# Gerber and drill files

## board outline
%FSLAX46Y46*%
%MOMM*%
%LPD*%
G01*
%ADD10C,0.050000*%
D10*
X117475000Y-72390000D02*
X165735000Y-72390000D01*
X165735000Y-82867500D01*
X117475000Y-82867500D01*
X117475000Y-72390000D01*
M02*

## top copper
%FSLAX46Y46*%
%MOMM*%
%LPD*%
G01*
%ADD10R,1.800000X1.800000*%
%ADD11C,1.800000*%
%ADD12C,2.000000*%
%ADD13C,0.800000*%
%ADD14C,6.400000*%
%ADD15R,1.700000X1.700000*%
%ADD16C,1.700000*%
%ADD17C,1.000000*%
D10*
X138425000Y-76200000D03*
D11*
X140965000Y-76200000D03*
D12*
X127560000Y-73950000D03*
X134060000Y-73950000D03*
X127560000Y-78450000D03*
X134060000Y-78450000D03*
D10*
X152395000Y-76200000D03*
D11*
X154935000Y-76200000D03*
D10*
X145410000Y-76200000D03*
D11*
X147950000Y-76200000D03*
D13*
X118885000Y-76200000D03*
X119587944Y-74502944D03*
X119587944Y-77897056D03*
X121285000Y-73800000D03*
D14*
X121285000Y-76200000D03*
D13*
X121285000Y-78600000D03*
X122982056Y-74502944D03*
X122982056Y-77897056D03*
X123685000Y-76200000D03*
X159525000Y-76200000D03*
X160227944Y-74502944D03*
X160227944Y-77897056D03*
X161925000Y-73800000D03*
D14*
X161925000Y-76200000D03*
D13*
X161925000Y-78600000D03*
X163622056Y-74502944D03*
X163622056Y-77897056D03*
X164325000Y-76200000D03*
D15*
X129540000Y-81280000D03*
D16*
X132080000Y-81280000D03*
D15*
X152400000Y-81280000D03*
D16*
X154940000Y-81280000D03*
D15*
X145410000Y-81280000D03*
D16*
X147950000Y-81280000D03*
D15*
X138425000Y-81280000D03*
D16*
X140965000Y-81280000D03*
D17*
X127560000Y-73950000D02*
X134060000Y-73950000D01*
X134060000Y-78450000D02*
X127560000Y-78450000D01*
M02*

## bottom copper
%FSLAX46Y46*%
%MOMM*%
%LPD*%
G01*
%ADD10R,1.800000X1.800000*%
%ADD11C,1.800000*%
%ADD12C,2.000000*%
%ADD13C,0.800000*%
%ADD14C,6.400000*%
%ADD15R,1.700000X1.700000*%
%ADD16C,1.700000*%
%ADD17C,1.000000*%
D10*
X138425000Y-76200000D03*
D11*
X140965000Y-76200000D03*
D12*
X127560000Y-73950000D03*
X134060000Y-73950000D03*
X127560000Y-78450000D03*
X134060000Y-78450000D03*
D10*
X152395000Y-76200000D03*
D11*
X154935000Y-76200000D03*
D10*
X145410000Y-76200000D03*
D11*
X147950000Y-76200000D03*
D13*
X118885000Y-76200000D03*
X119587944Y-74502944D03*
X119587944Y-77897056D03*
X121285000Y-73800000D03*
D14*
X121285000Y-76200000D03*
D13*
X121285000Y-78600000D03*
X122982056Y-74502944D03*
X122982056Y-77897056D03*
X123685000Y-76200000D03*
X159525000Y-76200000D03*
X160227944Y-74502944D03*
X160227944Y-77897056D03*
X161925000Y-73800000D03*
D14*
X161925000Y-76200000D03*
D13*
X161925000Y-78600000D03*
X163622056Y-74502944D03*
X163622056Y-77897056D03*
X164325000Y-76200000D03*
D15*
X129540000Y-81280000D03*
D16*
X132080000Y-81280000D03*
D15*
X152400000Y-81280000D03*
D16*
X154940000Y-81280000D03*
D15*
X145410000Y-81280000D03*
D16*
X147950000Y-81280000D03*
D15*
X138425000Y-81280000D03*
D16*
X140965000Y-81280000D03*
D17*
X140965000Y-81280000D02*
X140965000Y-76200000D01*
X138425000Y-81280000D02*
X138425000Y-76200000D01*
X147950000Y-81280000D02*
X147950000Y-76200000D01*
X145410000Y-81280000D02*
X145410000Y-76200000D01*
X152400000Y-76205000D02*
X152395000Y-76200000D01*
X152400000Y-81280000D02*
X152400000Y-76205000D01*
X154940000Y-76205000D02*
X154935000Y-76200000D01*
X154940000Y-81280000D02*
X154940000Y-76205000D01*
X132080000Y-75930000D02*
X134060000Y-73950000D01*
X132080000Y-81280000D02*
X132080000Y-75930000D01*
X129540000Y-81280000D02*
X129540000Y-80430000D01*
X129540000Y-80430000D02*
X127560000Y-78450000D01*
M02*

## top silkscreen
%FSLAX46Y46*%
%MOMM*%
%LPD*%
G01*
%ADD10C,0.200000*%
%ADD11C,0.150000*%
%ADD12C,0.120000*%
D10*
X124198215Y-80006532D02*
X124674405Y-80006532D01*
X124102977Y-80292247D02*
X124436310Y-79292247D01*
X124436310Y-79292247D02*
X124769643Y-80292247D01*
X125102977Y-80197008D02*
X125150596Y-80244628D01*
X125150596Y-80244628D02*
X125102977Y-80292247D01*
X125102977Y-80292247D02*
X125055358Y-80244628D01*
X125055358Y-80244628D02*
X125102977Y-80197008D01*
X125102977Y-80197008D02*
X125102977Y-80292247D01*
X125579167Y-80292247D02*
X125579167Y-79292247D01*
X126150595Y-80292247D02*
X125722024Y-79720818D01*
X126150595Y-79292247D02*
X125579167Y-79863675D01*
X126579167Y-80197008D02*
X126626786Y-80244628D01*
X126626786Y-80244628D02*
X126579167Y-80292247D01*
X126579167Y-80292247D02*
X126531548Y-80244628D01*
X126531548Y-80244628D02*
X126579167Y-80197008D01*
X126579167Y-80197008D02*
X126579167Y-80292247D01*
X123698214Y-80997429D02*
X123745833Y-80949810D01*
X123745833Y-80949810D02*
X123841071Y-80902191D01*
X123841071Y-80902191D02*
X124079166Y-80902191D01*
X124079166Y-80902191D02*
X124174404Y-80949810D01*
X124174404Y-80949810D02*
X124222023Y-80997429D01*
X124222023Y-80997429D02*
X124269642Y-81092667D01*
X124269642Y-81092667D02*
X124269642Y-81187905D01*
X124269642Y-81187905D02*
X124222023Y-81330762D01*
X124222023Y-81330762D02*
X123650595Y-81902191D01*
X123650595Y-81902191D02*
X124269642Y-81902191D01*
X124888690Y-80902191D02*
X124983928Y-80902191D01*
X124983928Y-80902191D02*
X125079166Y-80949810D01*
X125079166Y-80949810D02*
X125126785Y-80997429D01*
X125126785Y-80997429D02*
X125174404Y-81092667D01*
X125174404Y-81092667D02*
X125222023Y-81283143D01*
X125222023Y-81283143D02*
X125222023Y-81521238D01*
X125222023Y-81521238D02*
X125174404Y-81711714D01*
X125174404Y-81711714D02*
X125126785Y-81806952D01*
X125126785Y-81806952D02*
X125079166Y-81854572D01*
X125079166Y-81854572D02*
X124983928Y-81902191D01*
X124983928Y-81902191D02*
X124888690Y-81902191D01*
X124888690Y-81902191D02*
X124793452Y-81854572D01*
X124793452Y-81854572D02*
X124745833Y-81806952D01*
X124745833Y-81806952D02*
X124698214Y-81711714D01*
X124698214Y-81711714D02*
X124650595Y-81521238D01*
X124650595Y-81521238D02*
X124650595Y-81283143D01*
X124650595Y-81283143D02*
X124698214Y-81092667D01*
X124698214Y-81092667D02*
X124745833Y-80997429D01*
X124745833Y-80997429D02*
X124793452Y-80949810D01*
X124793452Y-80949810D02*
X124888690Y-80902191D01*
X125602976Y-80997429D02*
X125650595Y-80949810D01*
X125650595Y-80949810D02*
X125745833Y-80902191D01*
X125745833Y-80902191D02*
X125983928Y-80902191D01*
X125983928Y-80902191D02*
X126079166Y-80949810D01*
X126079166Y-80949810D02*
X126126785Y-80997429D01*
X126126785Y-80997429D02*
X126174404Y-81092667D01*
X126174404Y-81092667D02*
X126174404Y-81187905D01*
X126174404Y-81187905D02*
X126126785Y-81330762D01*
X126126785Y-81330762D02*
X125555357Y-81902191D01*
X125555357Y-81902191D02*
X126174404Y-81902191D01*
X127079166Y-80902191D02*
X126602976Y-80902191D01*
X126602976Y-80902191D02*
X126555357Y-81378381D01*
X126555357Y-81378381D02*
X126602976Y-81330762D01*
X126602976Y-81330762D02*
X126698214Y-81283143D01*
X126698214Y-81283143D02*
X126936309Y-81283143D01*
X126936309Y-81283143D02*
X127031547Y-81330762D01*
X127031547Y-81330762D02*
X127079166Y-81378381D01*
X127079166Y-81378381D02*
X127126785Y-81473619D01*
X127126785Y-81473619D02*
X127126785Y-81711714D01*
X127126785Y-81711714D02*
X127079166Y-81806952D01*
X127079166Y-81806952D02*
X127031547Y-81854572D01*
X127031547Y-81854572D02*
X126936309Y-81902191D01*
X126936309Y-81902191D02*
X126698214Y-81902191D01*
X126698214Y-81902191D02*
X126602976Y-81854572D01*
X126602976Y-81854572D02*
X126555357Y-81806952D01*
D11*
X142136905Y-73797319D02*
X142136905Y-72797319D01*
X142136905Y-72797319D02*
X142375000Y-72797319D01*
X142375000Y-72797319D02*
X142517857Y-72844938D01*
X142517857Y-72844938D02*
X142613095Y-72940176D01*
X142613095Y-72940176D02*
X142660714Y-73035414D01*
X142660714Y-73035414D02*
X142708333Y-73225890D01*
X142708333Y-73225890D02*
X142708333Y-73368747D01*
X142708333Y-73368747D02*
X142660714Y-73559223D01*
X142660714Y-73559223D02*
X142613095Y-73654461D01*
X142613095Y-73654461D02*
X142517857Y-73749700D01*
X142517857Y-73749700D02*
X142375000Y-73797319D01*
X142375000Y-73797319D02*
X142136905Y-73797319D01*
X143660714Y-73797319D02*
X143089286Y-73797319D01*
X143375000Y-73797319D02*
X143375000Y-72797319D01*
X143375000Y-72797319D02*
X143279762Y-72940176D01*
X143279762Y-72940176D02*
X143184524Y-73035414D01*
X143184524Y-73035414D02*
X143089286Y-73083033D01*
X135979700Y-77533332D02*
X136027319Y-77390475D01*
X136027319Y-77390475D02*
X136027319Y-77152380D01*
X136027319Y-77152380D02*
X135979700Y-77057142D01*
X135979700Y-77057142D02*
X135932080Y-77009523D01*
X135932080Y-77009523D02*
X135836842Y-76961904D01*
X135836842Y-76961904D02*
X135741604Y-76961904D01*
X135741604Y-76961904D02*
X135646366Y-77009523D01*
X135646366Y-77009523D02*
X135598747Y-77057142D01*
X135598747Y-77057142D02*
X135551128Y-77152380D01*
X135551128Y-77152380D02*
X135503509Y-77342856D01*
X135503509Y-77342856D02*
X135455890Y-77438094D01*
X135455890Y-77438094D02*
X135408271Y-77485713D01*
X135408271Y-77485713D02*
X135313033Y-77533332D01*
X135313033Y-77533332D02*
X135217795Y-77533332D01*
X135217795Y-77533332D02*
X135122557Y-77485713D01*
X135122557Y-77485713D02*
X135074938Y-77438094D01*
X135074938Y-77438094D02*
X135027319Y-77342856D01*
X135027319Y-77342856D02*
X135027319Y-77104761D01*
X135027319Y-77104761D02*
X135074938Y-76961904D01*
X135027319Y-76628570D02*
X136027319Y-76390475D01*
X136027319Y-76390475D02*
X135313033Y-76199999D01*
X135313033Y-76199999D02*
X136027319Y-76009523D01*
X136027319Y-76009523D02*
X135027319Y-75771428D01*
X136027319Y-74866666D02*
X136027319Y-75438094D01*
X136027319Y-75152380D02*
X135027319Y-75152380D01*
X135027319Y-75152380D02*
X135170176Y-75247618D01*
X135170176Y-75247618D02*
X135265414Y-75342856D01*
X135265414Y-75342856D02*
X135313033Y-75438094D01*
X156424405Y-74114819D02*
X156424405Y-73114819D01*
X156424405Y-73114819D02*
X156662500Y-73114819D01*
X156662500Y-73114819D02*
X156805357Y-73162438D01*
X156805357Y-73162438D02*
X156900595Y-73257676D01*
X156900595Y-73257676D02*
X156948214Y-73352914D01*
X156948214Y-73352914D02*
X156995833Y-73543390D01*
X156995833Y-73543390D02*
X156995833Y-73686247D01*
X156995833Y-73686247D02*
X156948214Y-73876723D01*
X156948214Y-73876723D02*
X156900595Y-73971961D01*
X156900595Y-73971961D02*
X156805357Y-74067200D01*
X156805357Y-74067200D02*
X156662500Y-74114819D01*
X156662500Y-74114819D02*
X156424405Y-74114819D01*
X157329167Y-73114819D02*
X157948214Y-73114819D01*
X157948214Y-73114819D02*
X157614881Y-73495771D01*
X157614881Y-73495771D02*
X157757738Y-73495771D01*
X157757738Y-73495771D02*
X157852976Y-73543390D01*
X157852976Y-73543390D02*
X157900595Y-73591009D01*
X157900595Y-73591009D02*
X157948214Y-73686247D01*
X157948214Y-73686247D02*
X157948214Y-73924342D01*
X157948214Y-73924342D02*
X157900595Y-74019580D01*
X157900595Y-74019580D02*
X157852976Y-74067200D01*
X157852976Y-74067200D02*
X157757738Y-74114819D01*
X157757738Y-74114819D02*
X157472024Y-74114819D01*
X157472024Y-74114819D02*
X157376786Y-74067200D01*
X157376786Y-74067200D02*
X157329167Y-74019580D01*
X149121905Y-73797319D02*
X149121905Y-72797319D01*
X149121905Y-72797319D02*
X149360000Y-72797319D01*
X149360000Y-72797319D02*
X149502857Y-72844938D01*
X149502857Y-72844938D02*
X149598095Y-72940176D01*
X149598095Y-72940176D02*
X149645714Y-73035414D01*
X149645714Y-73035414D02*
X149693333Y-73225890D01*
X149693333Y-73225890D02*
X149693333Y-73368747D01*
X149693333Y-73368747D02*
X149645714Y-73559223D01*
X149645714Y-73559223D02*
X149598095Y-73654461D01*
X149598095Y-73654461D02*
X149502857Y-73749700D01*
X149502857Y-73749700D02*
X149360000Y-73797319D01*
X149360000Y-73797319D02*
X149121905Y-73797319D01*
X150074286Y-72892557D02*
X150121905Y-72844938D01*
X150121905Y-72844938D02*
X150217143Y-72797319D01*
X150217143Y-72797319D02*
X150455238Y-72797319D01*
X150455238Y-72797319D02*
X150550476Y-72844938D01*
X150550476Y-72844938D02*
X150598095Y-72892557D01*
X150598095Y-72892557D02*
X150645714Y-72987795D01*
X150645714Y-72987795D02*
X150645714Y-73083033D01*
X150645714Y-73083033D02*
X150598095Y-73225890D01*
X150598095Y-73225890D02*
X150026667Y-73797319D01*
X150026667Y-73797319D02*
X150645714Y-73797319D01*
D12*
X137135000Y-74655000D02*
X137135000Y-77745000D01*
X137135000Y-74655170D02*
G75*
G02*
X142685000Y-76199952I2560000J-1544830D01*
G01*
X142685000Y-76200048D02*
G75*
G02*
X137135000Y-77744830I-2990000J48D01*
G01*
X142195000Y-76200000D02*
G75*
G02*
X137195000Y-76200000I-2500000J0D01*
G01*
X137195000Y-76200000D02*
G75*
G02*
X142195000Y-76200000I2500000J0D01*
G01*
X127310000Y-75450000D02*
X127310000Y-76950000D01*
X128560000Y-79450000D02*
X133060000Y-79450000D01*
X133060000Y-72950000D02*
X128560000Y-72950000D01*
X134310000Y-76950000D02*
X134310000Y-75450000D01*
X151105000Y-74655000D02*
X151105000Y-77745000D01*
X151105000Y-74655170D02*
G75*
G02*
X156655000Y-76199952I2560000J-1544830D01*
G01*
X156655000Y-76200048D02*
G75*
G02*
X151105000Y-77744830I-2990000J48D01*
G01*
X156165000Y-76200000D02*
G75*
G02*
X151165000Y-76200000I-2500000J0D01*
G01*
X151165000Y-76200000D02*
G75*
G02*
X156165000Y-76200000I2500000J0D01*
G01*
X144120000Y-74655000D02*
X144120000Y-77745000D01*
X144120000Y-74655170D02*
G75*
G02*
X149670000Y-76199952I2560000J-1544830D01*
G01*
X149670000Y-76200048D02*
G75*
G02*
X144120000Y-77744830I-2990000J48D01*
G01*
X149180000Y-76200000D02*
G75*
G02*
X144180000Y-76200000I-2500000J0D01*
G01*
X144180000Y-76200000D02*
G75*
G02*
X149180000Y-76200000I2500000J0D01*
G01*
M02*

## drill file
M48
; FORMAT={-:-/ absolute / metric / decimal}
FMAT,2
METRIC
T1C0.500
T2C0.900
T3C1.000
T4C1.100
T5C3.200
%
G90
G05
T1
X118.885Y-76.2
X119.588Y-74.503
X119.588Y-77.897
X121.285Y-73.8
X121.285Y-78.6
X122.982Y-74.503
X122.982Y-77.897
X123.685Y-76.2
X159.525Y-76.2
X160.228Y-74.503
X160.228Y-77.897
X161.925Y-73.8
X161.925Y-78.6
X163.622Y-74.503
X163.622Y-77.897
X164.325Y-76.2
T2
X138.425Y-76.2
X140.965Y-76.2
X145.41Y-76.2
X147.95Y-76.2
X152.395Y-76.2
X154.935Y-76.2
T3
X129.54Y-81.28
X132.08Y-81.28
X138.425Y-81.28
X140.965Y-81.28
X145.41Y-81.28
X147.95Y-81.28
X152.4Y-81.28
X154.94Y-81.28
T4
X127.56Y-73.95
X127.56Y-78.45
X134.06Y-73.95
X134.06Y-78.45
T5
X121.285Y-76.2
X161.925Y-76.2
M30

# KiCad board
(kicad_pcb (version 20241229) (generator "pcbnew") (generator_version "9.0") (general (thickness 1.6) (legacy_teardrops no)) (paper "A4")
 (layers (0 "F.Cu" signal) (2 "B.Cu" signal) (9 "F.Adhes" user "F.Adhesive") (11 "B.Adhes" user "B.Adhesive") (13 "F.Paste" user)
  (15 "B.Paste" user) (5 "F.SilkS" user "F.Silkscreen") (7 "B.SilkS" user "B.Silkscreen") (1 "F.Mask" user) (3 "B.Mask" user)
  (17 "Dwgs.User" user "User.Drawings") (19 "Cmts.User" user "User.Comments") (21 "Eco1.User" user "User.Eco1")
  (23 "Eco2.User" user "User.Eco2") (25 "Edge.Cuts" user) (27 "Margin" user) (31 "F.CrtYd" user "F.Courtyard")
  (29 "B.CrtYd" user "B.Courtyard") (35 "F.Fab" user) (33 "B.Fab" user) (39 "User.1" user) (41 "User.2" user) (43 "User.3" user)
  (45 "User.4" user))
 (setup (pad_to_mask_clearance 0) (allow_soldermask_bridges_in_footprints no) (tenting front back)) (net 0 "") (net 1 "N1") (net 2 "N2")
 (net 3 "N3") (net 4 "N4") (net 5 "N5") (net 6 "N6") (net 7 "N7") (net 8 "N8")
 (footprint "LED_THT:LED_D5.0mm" (layer "F.Cu") (at 138.425 76.2)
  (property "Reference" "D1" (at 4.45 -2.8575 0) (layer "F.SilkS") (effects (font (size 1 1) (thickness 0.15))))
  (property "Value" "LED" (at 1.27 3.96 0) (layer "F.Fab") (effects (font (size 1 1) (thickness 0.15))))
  (fp_line (start -1.29 -1.545) (end -1.29 1.545) (stroke (width 0.12) (type solid)) (layer "F.SilkS"))
  (fp_arc (start -1.29 -1.54483) (mid 2.071756 -2.880501) (end 4.26 -0.000048) (stroke (width 0.12) (type solid)) (layer "F.SilkS"))
  (fp_arc (start 4.26 0.000048) (mid 2.071756 2.880501) (end -1.29 1.54483) (stroke (width 0.12) (type solid)) (layer "F.SilkS"))
  (fp_circle (center 1.27 0) (end 3.77 0) (stroke (width 0.12) (type solid)) (fill no) (layer "F.SilkS"))
  (pad "1" thru_hole rect (at 0 0) (size 1.8 1.8) (drill 0.9) (layers "*.Cu" "*.Mask") (remove_unused_layers no) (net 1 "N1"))
  (pad "2" thru_hole circle (at 2.54 0) (size 1.8 1.8) (drill 0.9) (layers "*.Cu" "*.Mask") (remove_unused_layers no) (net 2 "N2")))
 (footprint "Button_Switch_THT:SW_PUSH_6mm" (layer "F.Cu") (at 127.56 73.95)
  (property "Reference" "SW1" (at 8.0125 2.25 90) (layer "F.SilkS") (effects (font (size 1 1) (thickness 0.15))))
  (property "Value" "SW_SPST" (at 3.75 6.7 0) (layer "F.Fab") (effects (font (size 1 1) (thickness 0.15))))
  (fp_line (start -0.25 1.5) (end -0.25 3) (stroke (width 0.12) (type solid)) (layer "F.SilkS"))
  (fp_line (start 1 5.5) (end 5.5 5.5) (stroke (width 0.12) (type solid)) (layer "F.SilkS"))
  (fp_line (start 5.5 -1) (end 1 -1) (stroke (width 0.12) (type solid)) (layer "F.SilkS"))
  (fp_line (start 6.75 3) (end 6.75 1.5) (stroke (width 0.12) (type solid)) (layer "F.SilkS"))
  (pad "1" thru_hole circle (at 0 0 90) (size 2 2) (drill 1.1) (layers "*.Cu" "*.Mask") (remove_unused_layers no) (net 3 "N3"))
  (pad "1" thru_hole circle (at 6.5 0 90) (size 2 2) (drill 1.1) (layers "*.Cu" "*.Mask") (remove_unused_layers no) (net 3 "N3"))
  (pad "2" thru_hole circle (at 0 4.5 90) (size 2 2) (drill 1.1) (layers "*.Cu" "*.Mask") (remove_unused_layers no) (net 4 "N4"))
  (pad "2" thru_hole circle (at 6.5 4.5 90) (size 2 2) (drill 1.1) (layers "*.Cu" "*.Mask") (remove_unused_layers no) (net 4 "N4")))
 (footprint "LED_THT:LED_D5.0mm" (layer "F.Cu") (at 152.395 76.2)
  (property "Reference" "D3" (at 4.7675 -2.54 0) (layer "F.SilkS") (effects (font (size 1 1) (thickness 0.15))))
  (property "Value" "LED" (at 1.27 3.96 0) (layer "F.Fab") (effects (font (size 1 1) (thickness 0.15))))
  (fp_line (start -1.29 -1.545) (end -1.29 1.545) (stroke (width 0.12) (type solid)) (layer "F.SilkS"))
  (fp_arc (start -1.29 -1.54483) (mid 2.071756 -2.880501) (end 4.26 -0.000048) (stroke (width 0.12) (type solid)) (layer "F.SilkS"))
  (fp_arc (start 4.26 0.000048) (mid 2.071756 2.880501) (end -1.29 1.54483) (stroke (width 0.12) (type solid)) (layer "F.SilkS"))
  (fp_circle (center 1.27 0) (end 3.77 0) (stroke (width 0.12) (type solid)) (fill no) (layer "F.SilkS"))
  (pad "1" thru_hole rect (at 0 0) (size 1.8 1.8) (drill 0.9) (layers "*.Cu" "*.Mask") (remove_unused_layers no) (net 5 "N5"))
  (pad "2" thru_hole circle (at 2.54 0) (size 1.8 1.8) (drill 0.9) (layers "*.Cu" "*.Mask") (remove_unused_layers no) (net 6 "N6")))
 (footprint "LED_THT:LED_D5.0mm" (layer "F.Cu") (at 145.41 76.2)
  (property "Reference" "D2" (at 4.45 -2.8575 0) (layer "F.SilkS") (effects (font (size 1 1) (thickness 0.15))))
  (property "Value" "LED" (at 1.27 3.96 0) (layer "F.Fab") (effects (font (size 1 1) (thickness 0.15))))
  (fp_line (start -1.29 -1.545) (end -1.29 1.545) (stroke (width 0.12) (type solid)) (layer "F.SilkS"))
  (fp_arc (start -1.29 -1.54483) (mid 2.071756 -2.880501) (end 4.26 -0.000048) (stroke (width 0.12) (type solid)) (layer "F.SilkS"))
  (fp_arc (start 4.26 0.000048) (mid 2.071756 2.880501) (end -1.29 1.54483) (stroke (width 0.12) (type solid)) (layer "F.SilkS"))
  (fp_circle (center 1.27 0) (end 3.77 0) (stroke (width 0.12) (type solid)) (fill no) (layer "F.SilkS"))
  (pad "1" thru_hole rect (at 0 0) (size 1.8 1.8) (drill 0.9) (layers "*.Cu" "*.Mask") (remove_unused_layers no) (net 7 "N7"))
  (pad "2" thru_hole circle (at 2.54 0) (size 1.8 1.8) (drill 0.9) (layers "*.Cu" "*.Mask") (remove_unused_layers no) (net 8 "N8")))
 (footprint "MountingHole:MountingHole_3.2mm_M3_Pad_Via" (layer "F.Cu") (at 121.285 76.2)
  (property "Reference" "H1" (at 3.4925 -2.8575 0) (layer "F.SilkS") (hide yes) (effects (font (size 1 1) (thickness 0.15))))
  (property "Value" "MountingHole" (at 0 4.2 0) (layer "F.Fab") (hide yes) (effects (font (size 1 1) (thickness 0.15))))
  (pad "1" thru_hole circle (at -2.4 0) (size 0.8 0.8) (drill 0.5) (layers "*.Cu" "*.Mask") (remove_unused_layers no) (zone_connect 2))
  (pad "1" thru_hole circle (at -1.697056 -1.697056) (size 0.8 0.8) (drill 0.5) (layers "*.Cu" "*.Mask") (remove_unused_layers no)
   (zone_connect 2))
  (pad "1" thru_hole circle (at -1.697056 1.697056) (size 0.8 0.8) (drill 0.5) (layers "*.Cu" "*.Mask") (remove_unused_layers no)
   (zone_connect 2))
  (pad "1" thru_hole circle (at 0 -2.4) (size 0.8 0.8) (drill 0.5) (layers "*.Cu" "*.Mask") (remove_unused_layers no) (zone_connect 2))
  (pad "1" thru_hole circle (at 0 0) (size 6.4 6.4) (drill 3.2) (layers "*.Cu" "*.Mask") (remove_unused_layers no))
  (pad "1" thru_hole circle (at 0 2.4) (size 0.8 0.8) (drill 0.5) (layers "*.Cu" "*.Mask") (remove_unused_layers no) (zone_connect 2))
  (pad "1" thru_hole circle (at 1.697056 -1.697056) (size 0.8 0.8) (drill 0.5) (layers "*.Cu" "*.Mask") (remove_unused_layers no)
   (zone_connect 2))
  (pad "1" thru_hole circle (at 1.697056 1.697056) (size 0.8 0.8) (drill 0.5) (layers "*.Cu" "*.Mask") (remove_unused_layers no)
   (zone_connect 2))
  (pad "1" thru_hole circle (at 2.4 0) (size 0.8 0.8) (drill 0.5) (layers "*.Cu" "*.Mask") (remove_unused_layers no) (zone_connect 2)))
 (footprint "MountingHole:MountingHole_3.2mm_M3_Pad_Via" (layer "F.Cu") (at 161.925 76.2)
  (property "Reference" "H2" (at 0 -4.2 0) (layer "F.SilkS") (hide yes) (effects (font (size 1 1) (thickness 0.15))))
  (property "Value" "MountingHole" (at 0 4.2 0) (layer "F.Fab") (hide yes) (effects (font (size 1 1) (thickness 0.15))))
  (pad "1" thru_hole circle (at -2.4 0) (size 0.8 0.8) (drill 0.5) (layers "*.Cu" "*.Mask") (remove_unused_layers no) (zone_connect 2))
  (pad "1" thru_hole circle (at -1.697056 -1.697056) (size 0.8 0.8) (drill 0.5) (layers "*.Cu" "*.Mask") (remove_unused_layers no)
   (zone_connect 2))
  (pad "1" thru_hole circle (at -1.697056 1.697056) (size 0.8 0.8) (drill 0.5) (layers "*.Cu" "*.Mask") (remove_unused_layers no)
   (zone_connect 2))
  (pad "1" thru_hole circle (at 0 -2.4) (size 0.8 0.8) (drill 0.5) (layers "*.Cu" "*.Mask") (remove_unused_layers no) (zone_connect 2))
  (pad "1" thru_hole circle (at 0 0) (size 6.4 6.4) (drill 3.2) (layers "*.Cu" "*.Mask") (remove_unused_layers no))
  (pad "1" thru_hole circle (at 0 2.4) (size 0.8 0.8) (drill 0.5) (layers "*.Cu" "*.Mask") (remove_unused_layers no) (zone_connect 2))
  (pad "1" thru_hole circle (at 1.697056 -1.697056) (size 0.8 0.8) (drill 0.5) (layers "*.Cu" "*.Mask") (remove_unused_layers no)
   (zone_connect 2))
  (pad "1" thru_hole circle (at 1.697056 1.697056) (size 0.8 0.8) (drill 0.5) (layers "*.Cu" "*.Mask") (remove_unused_layers no)
   (zone_connect 2))
  (pad "1" thru_hole circle (at 2.4 0) (size 0.8 0.8) (drill 0.5) (layers "*.Cu" "*.Mask") (remove_unused_layers no) (zone_connect 2)))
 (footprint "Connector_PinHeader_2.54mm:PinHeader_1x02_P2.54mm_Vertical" (layer "B.Cu") (at 129.54 81.28 -90)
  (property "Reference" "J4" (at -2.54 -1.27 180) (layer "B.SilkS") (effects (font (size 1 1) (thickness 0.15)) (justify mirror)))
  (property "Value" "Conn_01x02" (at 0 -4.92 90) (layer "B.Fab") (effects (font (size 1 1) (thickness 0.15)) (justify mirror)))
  (pad "1" thru_hole rect (at 0 0 270) (size 1.7 1.7) (drill 1) (layers "*.Cu" "*.Mask") (remove_unused_layers no) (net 4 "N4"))
  (pad "2" thru_hole circle (at 0 -2.54 270) (size 1.7 1.7) (drill 1) (layers "*.Cu" "*.Mask") (remove_unused_layers no) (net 3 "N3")))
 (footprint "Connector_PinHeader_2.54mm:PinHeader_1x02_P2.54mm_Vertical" (layer "B.Cu") (at 152.4 81.28 -90)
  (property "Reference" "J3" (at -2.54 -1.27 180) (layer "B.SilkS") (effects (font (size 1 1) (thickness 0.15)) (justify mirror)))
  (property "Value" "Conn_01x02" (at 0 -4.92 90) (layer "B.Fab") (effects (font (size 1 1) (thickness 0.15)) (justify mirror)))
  (pad "1" thru_hole rect (at 0 0 270) (size 1.7 1.7) (drill 1) (layers "*.Cu" "*.Mask") (remove_unused_layers no) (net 5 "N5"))
  (pad "2" thru_hole circle (at 0 -2.54 270) (size 1.7 1.7) (drill 1) (layers "*.Cu" "*.Mask") (remove_unused_layers no) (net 6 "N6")))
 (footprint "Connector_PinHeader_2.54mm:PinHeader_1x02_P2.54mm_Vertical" (layer "B.Cu") (at 145.41 81.28 -90)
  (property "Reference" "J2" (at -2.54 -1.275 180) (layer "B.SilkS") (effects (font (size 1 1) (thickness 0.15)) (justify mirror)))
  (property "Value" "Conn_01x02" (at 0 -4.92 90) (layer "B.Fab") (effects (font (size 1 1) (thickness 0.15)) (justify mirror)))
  (pad "1" thru_hole rect (at 0 0 270) (size 1.7 1.7) (drill 1) (layers "*.Cu" "*.Mask") (remove_unused_layers no) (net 7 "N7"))
  (pad "2" thru_hole circle (at 0 -2.54 270) (size 1.7 1.7) (drill 1) (layers "*.Cu" "*.Mask") (remove_unused_layers no) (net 8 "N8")))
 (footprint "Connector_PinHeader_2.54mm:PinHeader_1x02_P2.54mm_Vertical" (layer "B.Cu") (at 138.425 81.28 -90)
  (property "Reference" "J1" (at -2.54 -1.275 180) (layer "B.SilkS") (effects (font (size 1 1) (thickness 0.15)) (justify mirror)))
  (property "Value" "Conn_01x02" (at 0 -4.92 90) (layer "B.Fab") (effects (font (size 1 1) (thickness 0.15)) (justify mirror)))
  (pad "1" thru_hole rect (at 0 0 270) (size 1.7 1.7) (drill 1) (layers "*.Cu" "*.Mask") (remove_unused_layers no) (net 1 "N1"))
  (pad "2" thru_hole circle (at 0 -2.54 270) (size 1.7 1.7) (drill 1) (layers "*.Cu" "*.Mask") (remove_unused_layers no) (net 2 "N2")))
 (gr_rect (start 117.475 72.39) (end 165.735 82.8675) (stroke (width 0.05) (type default)) (fill no) (layer "Edge.Cuts"))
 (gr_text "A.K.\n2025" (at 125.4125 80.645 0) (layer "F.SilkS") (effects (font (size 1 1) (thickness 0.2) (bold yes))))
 (segment (start 140.965 81.28) (end 140.965 76.2) (width 1) (layer "B.Cu") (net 2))
 (segment (start 138.425 81.28) (end 138.425 76.2) (width 1) (layer "B.Cu") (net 1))
 (segment (start 147.95 81.28) (end 147.95 76.2) (width 1) (layer "B.Cu") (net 8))
 (segment (start 145.41 81.28) (end 145.41 76.2) (width 1) (layer "B.Cu") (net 7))
 (segment (start 152.4 76.205) (end 152.395 76.2) (width 1) (layer "B.Cu") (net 5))
 (segment (start 152.4 81.28) (end 152.4 76.205) (width 1) (layer "B.Cu") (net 5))
 (segment (start 154.94 76.205) (end 154.935 76.2) (width 1) (layer "B.Cu") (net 6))
 (segment (start 154.94 81.28) (end 154.94 76.205) (width 1) (layer "B.Cu") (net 6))
 (segment (start 127.56 73.95) (end 134.06 73.95) (width 1) (layer "F.Cu") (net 3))
 (segment (start 132.08 75.93) (end 134.06 73.95) (width 1) (layer "B.Cu") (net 3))
 (segment (start 132.08 81.28) (end 132.08 75.93) (width 1) (layer "B.Cu") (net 3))
 (segment (start 134.06 78.45) (end 127.56 78.45) (width 1) (layer "F.Cu") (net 4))
 (segment (start 129.54 81.28) (end 129.54 80.43) (width 1) (layer "B.Cu") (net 4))
 (segment (start 129.54 80.43) (end 127.56 78.45) (width 1) (layer "B.Cu") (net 4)))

